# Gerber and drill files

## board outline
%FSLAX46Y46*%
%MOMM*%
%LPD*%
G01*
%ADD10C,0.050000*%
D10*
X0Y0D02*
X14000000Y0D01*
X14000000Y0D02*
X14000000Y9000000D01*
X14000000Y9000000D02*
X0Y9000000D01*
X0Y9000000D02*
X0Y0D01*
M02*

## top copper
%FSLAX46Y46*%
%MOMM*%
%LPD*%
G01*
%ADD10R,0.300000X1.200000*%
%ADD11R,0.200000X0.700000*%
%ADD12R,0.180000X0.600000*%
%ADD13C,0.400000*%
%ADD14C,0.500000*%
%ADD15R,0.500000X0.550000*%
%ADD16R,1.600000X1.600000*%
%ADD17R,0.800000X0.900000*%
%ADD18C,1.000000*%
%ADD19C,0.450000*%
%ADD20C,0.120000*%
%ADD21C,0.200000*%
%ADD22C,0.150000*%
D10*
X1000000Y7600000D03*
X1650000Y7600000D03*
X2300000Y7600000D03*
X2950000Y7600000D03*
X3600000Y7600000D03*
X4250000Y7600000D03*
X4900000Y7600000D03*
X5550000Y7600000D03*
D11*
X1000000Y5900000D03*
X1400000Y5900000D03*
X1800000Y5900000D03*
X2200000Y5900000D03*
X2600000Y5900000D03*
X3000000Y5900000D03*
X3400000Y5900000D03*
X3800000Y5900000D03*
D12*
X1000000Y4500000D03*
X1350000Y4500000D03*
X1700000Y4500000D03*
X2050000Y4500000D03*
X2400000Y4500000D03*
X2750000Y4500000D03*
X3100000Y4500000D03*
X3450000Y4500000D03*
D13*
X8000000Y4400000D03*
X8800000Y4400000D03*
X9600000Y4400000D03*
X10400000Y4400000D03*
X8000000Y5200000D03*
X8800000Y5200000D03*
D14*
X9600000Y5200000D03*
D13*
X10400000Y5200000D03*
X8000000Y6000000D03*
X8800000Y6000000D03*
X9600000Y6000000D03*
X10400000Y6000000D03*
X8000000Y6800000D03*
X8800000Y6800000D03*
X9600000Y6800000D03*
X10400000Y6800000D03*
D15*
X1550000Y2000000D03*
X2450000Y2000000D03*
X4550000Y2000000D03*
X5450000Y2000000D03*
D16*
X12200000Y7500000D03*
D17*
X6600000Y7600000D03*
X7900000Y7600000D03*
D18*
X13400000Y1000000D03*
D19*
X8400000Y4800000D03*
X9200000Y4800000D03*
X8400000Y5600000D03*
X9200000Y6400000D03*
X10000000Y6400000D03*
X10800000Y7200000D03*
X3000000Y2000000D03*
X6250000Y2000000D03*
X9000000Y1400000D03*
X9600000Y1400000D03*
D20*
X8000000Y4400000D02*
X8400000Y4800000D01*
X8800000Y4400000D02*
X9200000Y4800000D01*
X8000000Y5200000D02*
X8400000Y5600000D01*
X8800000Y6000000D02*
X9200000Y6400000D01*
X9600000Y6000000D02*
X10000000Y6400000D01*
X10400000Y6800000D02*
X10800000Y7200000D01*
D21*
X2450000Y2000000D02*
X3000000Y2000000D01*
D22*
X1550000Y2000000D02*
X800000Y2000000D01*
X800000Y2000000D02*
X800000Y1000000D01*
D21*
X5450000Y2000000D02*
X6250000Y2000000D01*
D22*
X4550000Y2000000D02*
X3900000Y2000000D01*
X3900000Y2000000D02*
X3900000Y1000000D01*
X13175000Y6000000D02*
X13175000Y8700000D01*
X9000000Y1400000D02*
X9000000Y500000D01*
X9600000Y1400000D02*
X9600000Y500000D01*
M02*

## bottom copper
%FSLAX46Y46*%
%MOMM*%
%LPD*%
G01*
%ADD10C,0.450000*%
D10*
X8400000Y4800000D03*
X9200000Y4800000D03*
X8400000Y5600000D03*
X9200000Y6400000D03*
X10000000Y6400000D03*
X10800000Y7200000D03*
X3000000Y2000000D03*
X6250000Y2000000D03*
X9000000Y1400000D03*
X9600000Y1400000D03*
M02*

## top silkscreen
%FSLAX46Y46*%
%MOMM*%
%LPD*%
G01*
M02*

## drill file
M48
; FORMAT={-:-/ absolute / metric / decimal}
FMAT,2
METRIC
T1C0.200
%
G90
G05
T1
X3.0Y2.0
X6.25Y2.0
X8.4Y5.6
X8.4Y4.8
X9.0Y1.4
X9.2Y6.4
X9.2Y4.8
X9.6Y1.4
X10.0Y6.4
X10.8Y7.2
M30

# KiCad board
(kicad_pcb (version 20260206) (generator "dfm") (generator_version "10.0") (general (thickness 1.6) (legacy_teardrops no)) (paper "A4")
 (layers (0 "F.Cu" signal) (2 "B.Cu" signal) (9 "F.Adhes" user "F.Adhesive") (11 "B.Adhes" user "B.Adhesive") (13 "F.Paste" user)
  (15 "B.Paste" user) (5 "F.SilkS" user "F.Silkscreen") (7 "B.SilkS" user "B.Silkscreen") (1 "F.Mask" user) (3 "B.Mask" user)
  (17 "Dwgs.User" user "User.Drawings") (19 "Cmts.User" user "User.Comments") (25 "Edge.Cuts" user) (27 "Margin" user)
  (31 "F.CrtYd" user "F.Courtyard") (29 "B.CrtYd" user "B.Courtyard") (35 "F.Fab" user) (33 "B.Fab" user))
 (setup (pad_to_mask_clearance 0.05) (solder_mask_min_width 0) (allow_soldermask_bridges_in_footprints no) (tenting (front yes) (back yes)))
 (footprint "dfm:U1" (layer "F.Cu") (at 0 0 0)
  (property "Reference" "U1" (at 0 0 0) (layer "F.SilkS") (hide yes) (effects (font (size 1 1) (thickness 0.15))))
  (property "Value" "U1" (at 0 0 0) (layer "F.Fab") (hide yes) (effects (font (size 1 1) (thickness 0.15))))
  (pad "1" smd rect (at 1 -7.6 0) (size 0.3 1.2) (layers "F.Cu" "F.Mask" "F.Paste") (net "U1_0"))
  (pad "2" smd rect (at 1.65 -7.6 0) (size 0.3 1.2) (layers "F.Cu" "F.Mask" "F.Paste") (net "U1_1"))
  (pad "3" smd rect (at 2.3 -7.6 0) (size 0.3 1.2) (layers "F.Cu" "F.Mask" "F.Paste") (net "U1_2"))
  (pad "4" smd rect (at 2.95 -7.6 0) (size 0.3 1.2) (layers "F.Cu" "F.Mask" "F.Paste") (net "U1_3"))
  (pad "5" smd rect (at 3.6 -7.6 0) (size 0.3 1.2) (layers "F.Cu" "F.Mask" "F.Paste") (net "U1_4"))
  (pad "6" smd rect (at 4.25 -7.6 0) (size 0.3 1.2) (layers "F.Cu" "F.Mask" "F.Paste") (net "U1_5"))
  (pad "7" smd rect (at 4.9 -7.6 0) (size 0.3 1.2) (layers "F.Cu" "F.Mask" "F.Paste") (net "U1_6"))
  (pad "8" smd rect (at 5.55 -7.6 0) (size 0.3 1.2) (layers "F.Cu" "F.Mask" "F.Paste") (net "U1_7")))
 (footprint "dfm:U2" (layer "F.Cu") (at 0 0 0)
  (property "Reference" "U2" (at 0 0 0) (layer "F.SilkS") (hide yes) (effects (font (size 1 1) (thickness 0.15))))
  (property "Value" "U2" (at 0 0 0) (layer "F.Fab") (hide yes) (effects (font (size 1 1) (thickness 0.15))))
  (pad "1" smd rect (at 1 -5.9 0) (size 0.2 0.7) (layers "F.Cu" "F.Mask" "F.Paste") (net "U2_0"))
  (pad "2" smd rect (at 1.4 -5.9 0) (size 0.2 0.7) (layers "F.Cu" "F.Mask" "F.Paste") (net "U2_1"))
  (pad "3" smd rect (at 1.8 -5.9 0) (size 0.2 0.7) (layers "F.Cu" "F.Mask" "F.Paste") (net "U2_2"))
  (pad "4" smd rect (at 2.2 -5.9 0) (size 0.2 0.7) (layers "F.Cu" "F.Mask" "F.Paste") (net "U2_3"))
  (pad "5" smd rect (at 2.6 -5.9 0) (size 0.2 0.7) (layers "F.Cu" "F.Mask" "F.Paste") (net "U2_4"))
  (pad "6" smd rect (at 3 -5.9 0) (size 0.2 0.7) (layers "F.Cu" "F.Mask" "F.Paste") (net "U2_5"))
  (pad "7" smd rect (at 3.4 -5.9 0) (size 0.2 0.7) (layers "F.Cu" "F.Mask" "F.Paste") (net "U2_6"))
  (pad "8" smd rect (at 3.8 -5.9 0) (size 0.2 0.7) (layers "F.Cu" "F.Mask" "F.Paste") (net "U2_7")))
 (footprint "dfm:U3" (layer "F.Cu") (at 0 0 0)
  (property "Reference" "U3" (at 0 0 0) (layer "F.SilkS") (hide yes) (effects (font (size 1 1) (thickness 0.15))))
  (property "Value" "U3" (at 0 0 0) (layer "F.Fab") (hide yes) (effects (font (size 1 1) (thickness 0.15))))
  (pad "1" smd rect (at 1 -4.5 0) (size 0.18 0.6) (layers "F.Cu" "F.Mask" "F.Paste") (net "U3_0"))
  (pad "2" smd rect (at 1.35 -4.5 0) (size 0.18 0.6) (layers "F.Cu" "F.Mask" "F.Paste") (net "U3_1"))
  (pad "3" smd rect (at 1.7 -4.5 0) (size 0.18 0.6) (layers "F.Cu" "F.Mask" "F.Paste") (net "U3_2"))
  (pad "4" smd rect (at 2.05 -4.5 0) (size 0.18 0.6) (layers "F.Cu" "F.Mask" "F.Paste") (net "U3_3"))
  (pad "5" smd rect (at 2.4 -4.5 0) (size 0.18 0.6) (layers "F.Cu" "F.Mask" "F.Paste") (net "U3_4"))
  (pad "6" smd rect (at 2.75 -4.5 0) (size 0.18 0.6) (layers "F.Cu" "F.Mask" "F.Paste") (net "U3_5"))
  (pad "7" smd rect (at 3.1 -4.5 0) (size 0.18 0.6) (layers "F.Cu" "F.Mask" "F.Paste") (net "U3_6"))
  (pad "8" smd rect (at 3.45 -4.5 0) (size 0.18 0.6) (layers "F.Cu" "F.Mask" "F.Paste") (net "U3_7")))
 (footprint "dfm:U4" (layer "F.Cu") (at 0 0 0)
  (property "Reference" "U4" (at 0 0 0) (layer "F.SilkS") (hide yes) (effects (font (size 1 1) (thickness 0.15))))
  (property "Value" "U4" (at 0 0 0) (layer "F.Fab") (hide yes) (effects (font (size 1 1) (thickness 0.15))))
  (pad "1" smd circle (at 8 -4.4 0) (size 0.4 0.4) (layers "F.Cu" "F.Mask" "F.Paste") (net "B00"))
  (pad "2" smd circle (at 8.8 -4.4 0) (size 0.4 0.4) (layers "F.Cu" "F.Mask" "F.Paste") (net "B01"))
  (pad "3" smd circle (at 9.6 -4.4 0) (size 0.4 0.4) (layers "F.Cu" "F.Mask" "F.Paste") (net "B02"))
  (pad "4" smd circle (at 10.4 -4.4 0) (size 0.4 0.4) (layers "F.Cu" "F.Mask" "F.Paste") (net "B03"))
  (pad "5" smd circle (at 8 -5.2 0) (size 0.4 0.4) (layers "F.Cu" "F.Mask" "F.Paste") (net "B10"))
  (pad "6" smd circle (at 8.8 -5.2 0) (size 0.4 0.4) (layers "F.Cu" "F.Mask" "F.Paste") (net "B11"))
  (pad "7" smd circle (at 9.6 -5.2 0) (size 0.5 0.5) (layers "F.Cu" "F.Mask" "F.Paste") (solder_mask_margin -0.05) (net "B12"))
  (pad "8" smd circle (at 10.4 -5.2 0) (size 0.4 0.4) (layers "F.Cu" "F.Mask" "F.Paste") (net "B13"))
  (pad "9" smd circle (at 8 -6 0) (size 0.4 0.4) (layers "F.Cu" "F.Mask" "F.Paste") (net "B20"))
  (pad "10" smd circle (at 8.8 -6 0) (size 0.4 0.4) (layers "F.Cu" "F.Mask" "F.Paste") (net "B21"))
  (pad "11" smd circle (at 9.6 -6 0) (size 0.4 0.4) (layers "F.Cu" "F.Mask" "F.Paste") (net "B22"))
  (pad "12" smd circle (at 10.4 -6 0) (size 0.4 0.4) (layers "F.Cu" "F.Mask" "F.Paste") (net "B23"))
  (pad "13" smd circle (at 8 -6.8 0) (size 0.4 0.4) (layers "F.Cu" "F.Mask" "F.Paste") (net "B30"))
  (pad "14" smd circle (at 8.8 -6.8 0) (size 0.4 0.4) (layers "F.Cu" "F.Mask" "F.Paste") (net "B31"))
  (pad "15" smd circle (at 9.6 -6.8 0) (size 0.4 0.4) (layers "F.Cu" "F.Mask" "F.Paste") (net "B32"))
  (pad "16" smd circle (at 10.4 -6.8 0) (size 0.4 0.4) (layers "F.Cu" "F.Mask" "F.Paste") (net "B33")))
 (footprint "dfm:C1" (layer "F.Cu") (at 0 0 0)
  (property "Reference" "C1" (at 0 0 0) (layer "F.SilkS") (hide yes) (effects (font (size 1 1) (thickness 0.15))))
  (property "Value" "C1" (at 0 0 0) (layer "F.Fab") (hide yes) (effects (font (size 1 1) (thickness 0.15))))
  (pad "1" smd rect (at 1.55 -2 0) (size 0.5 0.55) (layers "F.Cu" "F.Mask" "F.Paste") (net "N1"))
  (pad "2" smd rect (at 2.45 -2 0) (size 0.5 0.55) (layers "F.Cu" "F.Mask" "F.Paste") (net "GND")))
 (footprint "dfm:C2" (layer "F.Cu") (at 0 0 0)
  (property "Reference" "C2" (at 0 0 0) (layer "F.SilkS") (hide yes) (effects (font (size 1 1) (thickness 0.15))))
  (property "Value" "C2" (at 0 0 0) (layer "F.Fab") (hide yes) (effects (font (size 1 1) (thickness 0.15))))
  (pad "1" smd rect (at 4.55 -2 0) (size 0.5 0.55) (layers "F.Cu" "F.Mask" "F.Paste") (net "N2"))
  (pad "2" smd rect (at 5.45 -2 0) (size 0.5 0.55) (layers "F.Cu" "F.Mask" "F.Paste") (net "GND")))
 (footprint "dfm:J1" (layer "F.Cu") (at 0 0 0)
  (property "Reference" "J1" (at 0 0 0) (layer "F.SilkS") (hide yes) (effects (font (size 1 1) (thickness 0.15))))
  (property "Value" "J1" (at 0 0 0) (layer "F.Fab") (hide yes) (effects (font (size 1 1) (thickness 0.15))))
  (pad "1" smd rect (at 12.2 -7.5 0) (size 1.6 1.6) (layers "F.Cu" "F.Mask" "F.Paste") (solder_mask_margin 0.15) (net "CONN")))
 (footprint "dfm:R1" (layer "F.Cu") (at 0 0 0)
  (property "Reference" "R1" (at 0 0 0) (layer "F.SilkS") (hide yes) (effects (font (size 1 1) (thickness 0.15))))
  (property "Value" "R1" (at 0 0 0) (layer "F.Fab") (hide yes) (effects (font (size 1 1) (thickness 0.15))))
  (pad "1" smd rect (at 6.6 -7.6 0) (size 0.8 0.9) (layers "F.Cu" "F.Mask" "F.Paste") (solder_mask_margin 0) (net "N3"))
  (pad "2" smd rect (at 7.9 -7.6 0) (size 0.8 0.9) (layers "F.Cu" "F.Mask" "F.Paste") (solder_mask_margin 0) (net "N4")))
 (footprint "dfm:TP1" (layer "F.Cu") (at 0 0 0)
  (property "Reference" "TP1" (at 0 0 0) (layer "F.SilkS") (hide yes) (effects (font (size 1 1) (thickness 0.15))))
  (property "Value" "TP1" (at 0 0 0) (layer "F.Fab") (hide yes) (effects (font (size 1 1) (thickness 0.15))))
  (pad "1" smd circle (at 13.4 -1 0) (size 1 1) (layers "F.Cu" "F.Mask" "F.Paste") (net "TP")))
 (gr_line (start 0 0) (end 14 0) (stroke (width 0.05) (type solid)) (layer "Edge.Cuts"))
 (gr_line (start 14 0) (end 14 -9) (stroke (width 0.05) (type solid)) (layer "Edge.Cuts"))
 (gr_line (start 14 -9) (end 0 -9) (stroke (width 0.05) (type solid)) (layer "Edge.Cuts"))
 (gr_line (start 0 -9) (end 0 0) (stroke (width 0.05) (type solid)) (layer "Edge.Cuts"))
 (via (at 8.4 -4.8) (size 0.45) (drill 0.2) (layers "F.Cu" "B.Cu") (tenting (front yes) (back yes)) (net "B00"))
 (segment (start 8 -4.4) (end 8.4 -4.8) (width 0.12) (layer "F.Cu") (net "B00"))
 (via (at 9.2 -4.8) (size 0.45) (drill 0.2) (layers "F.Cu" "B.Cu") (tenting (front yes) (back yes)) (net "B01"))
 (segment (start 8.8 -4.4) (end 9.2 -4.8) (width 0.12) (layer "F.Cu") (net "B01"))
 (via (at 8.4 -5.6) (size 0.45) (drill 0.2) (layers "F.Cu" "B.Cu") (tenting (front yes) (back yes)) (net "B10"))
 (segment (start 8 -5.2) (end 8.4 -5.6) (width 0.12) (layer "F.Cu") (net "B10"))
 (via (at 9.2 -6.4) (size 0.45) (drill 0.2) (layers "F.Cu" "B.Cu") (tenting (front no) (back yes)) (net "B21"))
 (segment (start 8.8 -6) (end 9.2 -6.4) (width 0.12) (layer "F.Cu") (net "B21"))
 (via (at 10 -6.4) (size 0.45) (drill 0.2) (layers "F.Cu" "B.Cu") (tenting (front yes) (back yes)) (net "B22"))
 (segment (start 9.6 -6) (end 10 -6.4) (width 0.12) (layer "F.Cu") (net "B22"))
 (via (at 10.8 -7.2) (size 0.45) (drill 0.2) (layers "F.Cu" "B.Cu") (tenting (front yes) (back yes)) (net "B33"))
 (segment (start 10.4 -6.8) (end 10.8 -7.2) (width 0.12) (layer "F.Cu") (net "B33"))
 (via (at 3 -2) (size 0.45) (drill 0.2) (layers "F.Cu" "B.Cu") (tenting (front no) (back yes)) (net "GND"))
 (segment (start 2.45 -2) (end 3 -2) (width 0.2) (layer "F.Cu") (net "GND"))
 (segment (start 1.55 -2) (end 0.8 -2) (width 0.15) (layer "F.Cu") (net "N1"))
 (segment (start 0.8 -2) (end 0.8 -1) (width 0.15) (layer "F.Cu") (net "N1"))
 (via (at 6.25 -2) (size 0.45) (drill 0.2) (layers "F.Cu" "B.Cu") (tenting (front yes) (back yes)) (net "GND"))
 (segment (start 5.45 -2) (end 6.25 -2) (width 0.2) (layer "F.Cu") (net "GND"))
 (segment (start 4.55 -2) (end 3.9 -2) (width 0.15) (layer "F.Cu") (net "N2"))
 (segment (start 3.9 -2) (end 3.9 -1) (width 0.15) (layer "F.Cu") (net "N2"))
 (segment (start 13.175 -6) (end 13.175 -8.7) (width 0.15) (layer "F.Cu") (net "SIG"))
 (via (at 9 -1.4) (size 0.45) (drill 0.2) (layers "F.Cu" "B.Cu") (tenting (front no) (back yes)) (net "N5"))
 (via (at 9.6 -1.4) (size 0.45) (drill 0.2) (layers "F.Cu" "B.Cu") (tenting (front no) (back yes)) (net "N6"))
 (segment (start 9 -1.4) (end 9 -0.5) (width 0.15) (layer "F.Cu") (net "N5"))
 (segment (start 9.6 -1.4) (end 9.6 -0.5) (width 0.15) (layer "F.Cu") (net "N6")))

